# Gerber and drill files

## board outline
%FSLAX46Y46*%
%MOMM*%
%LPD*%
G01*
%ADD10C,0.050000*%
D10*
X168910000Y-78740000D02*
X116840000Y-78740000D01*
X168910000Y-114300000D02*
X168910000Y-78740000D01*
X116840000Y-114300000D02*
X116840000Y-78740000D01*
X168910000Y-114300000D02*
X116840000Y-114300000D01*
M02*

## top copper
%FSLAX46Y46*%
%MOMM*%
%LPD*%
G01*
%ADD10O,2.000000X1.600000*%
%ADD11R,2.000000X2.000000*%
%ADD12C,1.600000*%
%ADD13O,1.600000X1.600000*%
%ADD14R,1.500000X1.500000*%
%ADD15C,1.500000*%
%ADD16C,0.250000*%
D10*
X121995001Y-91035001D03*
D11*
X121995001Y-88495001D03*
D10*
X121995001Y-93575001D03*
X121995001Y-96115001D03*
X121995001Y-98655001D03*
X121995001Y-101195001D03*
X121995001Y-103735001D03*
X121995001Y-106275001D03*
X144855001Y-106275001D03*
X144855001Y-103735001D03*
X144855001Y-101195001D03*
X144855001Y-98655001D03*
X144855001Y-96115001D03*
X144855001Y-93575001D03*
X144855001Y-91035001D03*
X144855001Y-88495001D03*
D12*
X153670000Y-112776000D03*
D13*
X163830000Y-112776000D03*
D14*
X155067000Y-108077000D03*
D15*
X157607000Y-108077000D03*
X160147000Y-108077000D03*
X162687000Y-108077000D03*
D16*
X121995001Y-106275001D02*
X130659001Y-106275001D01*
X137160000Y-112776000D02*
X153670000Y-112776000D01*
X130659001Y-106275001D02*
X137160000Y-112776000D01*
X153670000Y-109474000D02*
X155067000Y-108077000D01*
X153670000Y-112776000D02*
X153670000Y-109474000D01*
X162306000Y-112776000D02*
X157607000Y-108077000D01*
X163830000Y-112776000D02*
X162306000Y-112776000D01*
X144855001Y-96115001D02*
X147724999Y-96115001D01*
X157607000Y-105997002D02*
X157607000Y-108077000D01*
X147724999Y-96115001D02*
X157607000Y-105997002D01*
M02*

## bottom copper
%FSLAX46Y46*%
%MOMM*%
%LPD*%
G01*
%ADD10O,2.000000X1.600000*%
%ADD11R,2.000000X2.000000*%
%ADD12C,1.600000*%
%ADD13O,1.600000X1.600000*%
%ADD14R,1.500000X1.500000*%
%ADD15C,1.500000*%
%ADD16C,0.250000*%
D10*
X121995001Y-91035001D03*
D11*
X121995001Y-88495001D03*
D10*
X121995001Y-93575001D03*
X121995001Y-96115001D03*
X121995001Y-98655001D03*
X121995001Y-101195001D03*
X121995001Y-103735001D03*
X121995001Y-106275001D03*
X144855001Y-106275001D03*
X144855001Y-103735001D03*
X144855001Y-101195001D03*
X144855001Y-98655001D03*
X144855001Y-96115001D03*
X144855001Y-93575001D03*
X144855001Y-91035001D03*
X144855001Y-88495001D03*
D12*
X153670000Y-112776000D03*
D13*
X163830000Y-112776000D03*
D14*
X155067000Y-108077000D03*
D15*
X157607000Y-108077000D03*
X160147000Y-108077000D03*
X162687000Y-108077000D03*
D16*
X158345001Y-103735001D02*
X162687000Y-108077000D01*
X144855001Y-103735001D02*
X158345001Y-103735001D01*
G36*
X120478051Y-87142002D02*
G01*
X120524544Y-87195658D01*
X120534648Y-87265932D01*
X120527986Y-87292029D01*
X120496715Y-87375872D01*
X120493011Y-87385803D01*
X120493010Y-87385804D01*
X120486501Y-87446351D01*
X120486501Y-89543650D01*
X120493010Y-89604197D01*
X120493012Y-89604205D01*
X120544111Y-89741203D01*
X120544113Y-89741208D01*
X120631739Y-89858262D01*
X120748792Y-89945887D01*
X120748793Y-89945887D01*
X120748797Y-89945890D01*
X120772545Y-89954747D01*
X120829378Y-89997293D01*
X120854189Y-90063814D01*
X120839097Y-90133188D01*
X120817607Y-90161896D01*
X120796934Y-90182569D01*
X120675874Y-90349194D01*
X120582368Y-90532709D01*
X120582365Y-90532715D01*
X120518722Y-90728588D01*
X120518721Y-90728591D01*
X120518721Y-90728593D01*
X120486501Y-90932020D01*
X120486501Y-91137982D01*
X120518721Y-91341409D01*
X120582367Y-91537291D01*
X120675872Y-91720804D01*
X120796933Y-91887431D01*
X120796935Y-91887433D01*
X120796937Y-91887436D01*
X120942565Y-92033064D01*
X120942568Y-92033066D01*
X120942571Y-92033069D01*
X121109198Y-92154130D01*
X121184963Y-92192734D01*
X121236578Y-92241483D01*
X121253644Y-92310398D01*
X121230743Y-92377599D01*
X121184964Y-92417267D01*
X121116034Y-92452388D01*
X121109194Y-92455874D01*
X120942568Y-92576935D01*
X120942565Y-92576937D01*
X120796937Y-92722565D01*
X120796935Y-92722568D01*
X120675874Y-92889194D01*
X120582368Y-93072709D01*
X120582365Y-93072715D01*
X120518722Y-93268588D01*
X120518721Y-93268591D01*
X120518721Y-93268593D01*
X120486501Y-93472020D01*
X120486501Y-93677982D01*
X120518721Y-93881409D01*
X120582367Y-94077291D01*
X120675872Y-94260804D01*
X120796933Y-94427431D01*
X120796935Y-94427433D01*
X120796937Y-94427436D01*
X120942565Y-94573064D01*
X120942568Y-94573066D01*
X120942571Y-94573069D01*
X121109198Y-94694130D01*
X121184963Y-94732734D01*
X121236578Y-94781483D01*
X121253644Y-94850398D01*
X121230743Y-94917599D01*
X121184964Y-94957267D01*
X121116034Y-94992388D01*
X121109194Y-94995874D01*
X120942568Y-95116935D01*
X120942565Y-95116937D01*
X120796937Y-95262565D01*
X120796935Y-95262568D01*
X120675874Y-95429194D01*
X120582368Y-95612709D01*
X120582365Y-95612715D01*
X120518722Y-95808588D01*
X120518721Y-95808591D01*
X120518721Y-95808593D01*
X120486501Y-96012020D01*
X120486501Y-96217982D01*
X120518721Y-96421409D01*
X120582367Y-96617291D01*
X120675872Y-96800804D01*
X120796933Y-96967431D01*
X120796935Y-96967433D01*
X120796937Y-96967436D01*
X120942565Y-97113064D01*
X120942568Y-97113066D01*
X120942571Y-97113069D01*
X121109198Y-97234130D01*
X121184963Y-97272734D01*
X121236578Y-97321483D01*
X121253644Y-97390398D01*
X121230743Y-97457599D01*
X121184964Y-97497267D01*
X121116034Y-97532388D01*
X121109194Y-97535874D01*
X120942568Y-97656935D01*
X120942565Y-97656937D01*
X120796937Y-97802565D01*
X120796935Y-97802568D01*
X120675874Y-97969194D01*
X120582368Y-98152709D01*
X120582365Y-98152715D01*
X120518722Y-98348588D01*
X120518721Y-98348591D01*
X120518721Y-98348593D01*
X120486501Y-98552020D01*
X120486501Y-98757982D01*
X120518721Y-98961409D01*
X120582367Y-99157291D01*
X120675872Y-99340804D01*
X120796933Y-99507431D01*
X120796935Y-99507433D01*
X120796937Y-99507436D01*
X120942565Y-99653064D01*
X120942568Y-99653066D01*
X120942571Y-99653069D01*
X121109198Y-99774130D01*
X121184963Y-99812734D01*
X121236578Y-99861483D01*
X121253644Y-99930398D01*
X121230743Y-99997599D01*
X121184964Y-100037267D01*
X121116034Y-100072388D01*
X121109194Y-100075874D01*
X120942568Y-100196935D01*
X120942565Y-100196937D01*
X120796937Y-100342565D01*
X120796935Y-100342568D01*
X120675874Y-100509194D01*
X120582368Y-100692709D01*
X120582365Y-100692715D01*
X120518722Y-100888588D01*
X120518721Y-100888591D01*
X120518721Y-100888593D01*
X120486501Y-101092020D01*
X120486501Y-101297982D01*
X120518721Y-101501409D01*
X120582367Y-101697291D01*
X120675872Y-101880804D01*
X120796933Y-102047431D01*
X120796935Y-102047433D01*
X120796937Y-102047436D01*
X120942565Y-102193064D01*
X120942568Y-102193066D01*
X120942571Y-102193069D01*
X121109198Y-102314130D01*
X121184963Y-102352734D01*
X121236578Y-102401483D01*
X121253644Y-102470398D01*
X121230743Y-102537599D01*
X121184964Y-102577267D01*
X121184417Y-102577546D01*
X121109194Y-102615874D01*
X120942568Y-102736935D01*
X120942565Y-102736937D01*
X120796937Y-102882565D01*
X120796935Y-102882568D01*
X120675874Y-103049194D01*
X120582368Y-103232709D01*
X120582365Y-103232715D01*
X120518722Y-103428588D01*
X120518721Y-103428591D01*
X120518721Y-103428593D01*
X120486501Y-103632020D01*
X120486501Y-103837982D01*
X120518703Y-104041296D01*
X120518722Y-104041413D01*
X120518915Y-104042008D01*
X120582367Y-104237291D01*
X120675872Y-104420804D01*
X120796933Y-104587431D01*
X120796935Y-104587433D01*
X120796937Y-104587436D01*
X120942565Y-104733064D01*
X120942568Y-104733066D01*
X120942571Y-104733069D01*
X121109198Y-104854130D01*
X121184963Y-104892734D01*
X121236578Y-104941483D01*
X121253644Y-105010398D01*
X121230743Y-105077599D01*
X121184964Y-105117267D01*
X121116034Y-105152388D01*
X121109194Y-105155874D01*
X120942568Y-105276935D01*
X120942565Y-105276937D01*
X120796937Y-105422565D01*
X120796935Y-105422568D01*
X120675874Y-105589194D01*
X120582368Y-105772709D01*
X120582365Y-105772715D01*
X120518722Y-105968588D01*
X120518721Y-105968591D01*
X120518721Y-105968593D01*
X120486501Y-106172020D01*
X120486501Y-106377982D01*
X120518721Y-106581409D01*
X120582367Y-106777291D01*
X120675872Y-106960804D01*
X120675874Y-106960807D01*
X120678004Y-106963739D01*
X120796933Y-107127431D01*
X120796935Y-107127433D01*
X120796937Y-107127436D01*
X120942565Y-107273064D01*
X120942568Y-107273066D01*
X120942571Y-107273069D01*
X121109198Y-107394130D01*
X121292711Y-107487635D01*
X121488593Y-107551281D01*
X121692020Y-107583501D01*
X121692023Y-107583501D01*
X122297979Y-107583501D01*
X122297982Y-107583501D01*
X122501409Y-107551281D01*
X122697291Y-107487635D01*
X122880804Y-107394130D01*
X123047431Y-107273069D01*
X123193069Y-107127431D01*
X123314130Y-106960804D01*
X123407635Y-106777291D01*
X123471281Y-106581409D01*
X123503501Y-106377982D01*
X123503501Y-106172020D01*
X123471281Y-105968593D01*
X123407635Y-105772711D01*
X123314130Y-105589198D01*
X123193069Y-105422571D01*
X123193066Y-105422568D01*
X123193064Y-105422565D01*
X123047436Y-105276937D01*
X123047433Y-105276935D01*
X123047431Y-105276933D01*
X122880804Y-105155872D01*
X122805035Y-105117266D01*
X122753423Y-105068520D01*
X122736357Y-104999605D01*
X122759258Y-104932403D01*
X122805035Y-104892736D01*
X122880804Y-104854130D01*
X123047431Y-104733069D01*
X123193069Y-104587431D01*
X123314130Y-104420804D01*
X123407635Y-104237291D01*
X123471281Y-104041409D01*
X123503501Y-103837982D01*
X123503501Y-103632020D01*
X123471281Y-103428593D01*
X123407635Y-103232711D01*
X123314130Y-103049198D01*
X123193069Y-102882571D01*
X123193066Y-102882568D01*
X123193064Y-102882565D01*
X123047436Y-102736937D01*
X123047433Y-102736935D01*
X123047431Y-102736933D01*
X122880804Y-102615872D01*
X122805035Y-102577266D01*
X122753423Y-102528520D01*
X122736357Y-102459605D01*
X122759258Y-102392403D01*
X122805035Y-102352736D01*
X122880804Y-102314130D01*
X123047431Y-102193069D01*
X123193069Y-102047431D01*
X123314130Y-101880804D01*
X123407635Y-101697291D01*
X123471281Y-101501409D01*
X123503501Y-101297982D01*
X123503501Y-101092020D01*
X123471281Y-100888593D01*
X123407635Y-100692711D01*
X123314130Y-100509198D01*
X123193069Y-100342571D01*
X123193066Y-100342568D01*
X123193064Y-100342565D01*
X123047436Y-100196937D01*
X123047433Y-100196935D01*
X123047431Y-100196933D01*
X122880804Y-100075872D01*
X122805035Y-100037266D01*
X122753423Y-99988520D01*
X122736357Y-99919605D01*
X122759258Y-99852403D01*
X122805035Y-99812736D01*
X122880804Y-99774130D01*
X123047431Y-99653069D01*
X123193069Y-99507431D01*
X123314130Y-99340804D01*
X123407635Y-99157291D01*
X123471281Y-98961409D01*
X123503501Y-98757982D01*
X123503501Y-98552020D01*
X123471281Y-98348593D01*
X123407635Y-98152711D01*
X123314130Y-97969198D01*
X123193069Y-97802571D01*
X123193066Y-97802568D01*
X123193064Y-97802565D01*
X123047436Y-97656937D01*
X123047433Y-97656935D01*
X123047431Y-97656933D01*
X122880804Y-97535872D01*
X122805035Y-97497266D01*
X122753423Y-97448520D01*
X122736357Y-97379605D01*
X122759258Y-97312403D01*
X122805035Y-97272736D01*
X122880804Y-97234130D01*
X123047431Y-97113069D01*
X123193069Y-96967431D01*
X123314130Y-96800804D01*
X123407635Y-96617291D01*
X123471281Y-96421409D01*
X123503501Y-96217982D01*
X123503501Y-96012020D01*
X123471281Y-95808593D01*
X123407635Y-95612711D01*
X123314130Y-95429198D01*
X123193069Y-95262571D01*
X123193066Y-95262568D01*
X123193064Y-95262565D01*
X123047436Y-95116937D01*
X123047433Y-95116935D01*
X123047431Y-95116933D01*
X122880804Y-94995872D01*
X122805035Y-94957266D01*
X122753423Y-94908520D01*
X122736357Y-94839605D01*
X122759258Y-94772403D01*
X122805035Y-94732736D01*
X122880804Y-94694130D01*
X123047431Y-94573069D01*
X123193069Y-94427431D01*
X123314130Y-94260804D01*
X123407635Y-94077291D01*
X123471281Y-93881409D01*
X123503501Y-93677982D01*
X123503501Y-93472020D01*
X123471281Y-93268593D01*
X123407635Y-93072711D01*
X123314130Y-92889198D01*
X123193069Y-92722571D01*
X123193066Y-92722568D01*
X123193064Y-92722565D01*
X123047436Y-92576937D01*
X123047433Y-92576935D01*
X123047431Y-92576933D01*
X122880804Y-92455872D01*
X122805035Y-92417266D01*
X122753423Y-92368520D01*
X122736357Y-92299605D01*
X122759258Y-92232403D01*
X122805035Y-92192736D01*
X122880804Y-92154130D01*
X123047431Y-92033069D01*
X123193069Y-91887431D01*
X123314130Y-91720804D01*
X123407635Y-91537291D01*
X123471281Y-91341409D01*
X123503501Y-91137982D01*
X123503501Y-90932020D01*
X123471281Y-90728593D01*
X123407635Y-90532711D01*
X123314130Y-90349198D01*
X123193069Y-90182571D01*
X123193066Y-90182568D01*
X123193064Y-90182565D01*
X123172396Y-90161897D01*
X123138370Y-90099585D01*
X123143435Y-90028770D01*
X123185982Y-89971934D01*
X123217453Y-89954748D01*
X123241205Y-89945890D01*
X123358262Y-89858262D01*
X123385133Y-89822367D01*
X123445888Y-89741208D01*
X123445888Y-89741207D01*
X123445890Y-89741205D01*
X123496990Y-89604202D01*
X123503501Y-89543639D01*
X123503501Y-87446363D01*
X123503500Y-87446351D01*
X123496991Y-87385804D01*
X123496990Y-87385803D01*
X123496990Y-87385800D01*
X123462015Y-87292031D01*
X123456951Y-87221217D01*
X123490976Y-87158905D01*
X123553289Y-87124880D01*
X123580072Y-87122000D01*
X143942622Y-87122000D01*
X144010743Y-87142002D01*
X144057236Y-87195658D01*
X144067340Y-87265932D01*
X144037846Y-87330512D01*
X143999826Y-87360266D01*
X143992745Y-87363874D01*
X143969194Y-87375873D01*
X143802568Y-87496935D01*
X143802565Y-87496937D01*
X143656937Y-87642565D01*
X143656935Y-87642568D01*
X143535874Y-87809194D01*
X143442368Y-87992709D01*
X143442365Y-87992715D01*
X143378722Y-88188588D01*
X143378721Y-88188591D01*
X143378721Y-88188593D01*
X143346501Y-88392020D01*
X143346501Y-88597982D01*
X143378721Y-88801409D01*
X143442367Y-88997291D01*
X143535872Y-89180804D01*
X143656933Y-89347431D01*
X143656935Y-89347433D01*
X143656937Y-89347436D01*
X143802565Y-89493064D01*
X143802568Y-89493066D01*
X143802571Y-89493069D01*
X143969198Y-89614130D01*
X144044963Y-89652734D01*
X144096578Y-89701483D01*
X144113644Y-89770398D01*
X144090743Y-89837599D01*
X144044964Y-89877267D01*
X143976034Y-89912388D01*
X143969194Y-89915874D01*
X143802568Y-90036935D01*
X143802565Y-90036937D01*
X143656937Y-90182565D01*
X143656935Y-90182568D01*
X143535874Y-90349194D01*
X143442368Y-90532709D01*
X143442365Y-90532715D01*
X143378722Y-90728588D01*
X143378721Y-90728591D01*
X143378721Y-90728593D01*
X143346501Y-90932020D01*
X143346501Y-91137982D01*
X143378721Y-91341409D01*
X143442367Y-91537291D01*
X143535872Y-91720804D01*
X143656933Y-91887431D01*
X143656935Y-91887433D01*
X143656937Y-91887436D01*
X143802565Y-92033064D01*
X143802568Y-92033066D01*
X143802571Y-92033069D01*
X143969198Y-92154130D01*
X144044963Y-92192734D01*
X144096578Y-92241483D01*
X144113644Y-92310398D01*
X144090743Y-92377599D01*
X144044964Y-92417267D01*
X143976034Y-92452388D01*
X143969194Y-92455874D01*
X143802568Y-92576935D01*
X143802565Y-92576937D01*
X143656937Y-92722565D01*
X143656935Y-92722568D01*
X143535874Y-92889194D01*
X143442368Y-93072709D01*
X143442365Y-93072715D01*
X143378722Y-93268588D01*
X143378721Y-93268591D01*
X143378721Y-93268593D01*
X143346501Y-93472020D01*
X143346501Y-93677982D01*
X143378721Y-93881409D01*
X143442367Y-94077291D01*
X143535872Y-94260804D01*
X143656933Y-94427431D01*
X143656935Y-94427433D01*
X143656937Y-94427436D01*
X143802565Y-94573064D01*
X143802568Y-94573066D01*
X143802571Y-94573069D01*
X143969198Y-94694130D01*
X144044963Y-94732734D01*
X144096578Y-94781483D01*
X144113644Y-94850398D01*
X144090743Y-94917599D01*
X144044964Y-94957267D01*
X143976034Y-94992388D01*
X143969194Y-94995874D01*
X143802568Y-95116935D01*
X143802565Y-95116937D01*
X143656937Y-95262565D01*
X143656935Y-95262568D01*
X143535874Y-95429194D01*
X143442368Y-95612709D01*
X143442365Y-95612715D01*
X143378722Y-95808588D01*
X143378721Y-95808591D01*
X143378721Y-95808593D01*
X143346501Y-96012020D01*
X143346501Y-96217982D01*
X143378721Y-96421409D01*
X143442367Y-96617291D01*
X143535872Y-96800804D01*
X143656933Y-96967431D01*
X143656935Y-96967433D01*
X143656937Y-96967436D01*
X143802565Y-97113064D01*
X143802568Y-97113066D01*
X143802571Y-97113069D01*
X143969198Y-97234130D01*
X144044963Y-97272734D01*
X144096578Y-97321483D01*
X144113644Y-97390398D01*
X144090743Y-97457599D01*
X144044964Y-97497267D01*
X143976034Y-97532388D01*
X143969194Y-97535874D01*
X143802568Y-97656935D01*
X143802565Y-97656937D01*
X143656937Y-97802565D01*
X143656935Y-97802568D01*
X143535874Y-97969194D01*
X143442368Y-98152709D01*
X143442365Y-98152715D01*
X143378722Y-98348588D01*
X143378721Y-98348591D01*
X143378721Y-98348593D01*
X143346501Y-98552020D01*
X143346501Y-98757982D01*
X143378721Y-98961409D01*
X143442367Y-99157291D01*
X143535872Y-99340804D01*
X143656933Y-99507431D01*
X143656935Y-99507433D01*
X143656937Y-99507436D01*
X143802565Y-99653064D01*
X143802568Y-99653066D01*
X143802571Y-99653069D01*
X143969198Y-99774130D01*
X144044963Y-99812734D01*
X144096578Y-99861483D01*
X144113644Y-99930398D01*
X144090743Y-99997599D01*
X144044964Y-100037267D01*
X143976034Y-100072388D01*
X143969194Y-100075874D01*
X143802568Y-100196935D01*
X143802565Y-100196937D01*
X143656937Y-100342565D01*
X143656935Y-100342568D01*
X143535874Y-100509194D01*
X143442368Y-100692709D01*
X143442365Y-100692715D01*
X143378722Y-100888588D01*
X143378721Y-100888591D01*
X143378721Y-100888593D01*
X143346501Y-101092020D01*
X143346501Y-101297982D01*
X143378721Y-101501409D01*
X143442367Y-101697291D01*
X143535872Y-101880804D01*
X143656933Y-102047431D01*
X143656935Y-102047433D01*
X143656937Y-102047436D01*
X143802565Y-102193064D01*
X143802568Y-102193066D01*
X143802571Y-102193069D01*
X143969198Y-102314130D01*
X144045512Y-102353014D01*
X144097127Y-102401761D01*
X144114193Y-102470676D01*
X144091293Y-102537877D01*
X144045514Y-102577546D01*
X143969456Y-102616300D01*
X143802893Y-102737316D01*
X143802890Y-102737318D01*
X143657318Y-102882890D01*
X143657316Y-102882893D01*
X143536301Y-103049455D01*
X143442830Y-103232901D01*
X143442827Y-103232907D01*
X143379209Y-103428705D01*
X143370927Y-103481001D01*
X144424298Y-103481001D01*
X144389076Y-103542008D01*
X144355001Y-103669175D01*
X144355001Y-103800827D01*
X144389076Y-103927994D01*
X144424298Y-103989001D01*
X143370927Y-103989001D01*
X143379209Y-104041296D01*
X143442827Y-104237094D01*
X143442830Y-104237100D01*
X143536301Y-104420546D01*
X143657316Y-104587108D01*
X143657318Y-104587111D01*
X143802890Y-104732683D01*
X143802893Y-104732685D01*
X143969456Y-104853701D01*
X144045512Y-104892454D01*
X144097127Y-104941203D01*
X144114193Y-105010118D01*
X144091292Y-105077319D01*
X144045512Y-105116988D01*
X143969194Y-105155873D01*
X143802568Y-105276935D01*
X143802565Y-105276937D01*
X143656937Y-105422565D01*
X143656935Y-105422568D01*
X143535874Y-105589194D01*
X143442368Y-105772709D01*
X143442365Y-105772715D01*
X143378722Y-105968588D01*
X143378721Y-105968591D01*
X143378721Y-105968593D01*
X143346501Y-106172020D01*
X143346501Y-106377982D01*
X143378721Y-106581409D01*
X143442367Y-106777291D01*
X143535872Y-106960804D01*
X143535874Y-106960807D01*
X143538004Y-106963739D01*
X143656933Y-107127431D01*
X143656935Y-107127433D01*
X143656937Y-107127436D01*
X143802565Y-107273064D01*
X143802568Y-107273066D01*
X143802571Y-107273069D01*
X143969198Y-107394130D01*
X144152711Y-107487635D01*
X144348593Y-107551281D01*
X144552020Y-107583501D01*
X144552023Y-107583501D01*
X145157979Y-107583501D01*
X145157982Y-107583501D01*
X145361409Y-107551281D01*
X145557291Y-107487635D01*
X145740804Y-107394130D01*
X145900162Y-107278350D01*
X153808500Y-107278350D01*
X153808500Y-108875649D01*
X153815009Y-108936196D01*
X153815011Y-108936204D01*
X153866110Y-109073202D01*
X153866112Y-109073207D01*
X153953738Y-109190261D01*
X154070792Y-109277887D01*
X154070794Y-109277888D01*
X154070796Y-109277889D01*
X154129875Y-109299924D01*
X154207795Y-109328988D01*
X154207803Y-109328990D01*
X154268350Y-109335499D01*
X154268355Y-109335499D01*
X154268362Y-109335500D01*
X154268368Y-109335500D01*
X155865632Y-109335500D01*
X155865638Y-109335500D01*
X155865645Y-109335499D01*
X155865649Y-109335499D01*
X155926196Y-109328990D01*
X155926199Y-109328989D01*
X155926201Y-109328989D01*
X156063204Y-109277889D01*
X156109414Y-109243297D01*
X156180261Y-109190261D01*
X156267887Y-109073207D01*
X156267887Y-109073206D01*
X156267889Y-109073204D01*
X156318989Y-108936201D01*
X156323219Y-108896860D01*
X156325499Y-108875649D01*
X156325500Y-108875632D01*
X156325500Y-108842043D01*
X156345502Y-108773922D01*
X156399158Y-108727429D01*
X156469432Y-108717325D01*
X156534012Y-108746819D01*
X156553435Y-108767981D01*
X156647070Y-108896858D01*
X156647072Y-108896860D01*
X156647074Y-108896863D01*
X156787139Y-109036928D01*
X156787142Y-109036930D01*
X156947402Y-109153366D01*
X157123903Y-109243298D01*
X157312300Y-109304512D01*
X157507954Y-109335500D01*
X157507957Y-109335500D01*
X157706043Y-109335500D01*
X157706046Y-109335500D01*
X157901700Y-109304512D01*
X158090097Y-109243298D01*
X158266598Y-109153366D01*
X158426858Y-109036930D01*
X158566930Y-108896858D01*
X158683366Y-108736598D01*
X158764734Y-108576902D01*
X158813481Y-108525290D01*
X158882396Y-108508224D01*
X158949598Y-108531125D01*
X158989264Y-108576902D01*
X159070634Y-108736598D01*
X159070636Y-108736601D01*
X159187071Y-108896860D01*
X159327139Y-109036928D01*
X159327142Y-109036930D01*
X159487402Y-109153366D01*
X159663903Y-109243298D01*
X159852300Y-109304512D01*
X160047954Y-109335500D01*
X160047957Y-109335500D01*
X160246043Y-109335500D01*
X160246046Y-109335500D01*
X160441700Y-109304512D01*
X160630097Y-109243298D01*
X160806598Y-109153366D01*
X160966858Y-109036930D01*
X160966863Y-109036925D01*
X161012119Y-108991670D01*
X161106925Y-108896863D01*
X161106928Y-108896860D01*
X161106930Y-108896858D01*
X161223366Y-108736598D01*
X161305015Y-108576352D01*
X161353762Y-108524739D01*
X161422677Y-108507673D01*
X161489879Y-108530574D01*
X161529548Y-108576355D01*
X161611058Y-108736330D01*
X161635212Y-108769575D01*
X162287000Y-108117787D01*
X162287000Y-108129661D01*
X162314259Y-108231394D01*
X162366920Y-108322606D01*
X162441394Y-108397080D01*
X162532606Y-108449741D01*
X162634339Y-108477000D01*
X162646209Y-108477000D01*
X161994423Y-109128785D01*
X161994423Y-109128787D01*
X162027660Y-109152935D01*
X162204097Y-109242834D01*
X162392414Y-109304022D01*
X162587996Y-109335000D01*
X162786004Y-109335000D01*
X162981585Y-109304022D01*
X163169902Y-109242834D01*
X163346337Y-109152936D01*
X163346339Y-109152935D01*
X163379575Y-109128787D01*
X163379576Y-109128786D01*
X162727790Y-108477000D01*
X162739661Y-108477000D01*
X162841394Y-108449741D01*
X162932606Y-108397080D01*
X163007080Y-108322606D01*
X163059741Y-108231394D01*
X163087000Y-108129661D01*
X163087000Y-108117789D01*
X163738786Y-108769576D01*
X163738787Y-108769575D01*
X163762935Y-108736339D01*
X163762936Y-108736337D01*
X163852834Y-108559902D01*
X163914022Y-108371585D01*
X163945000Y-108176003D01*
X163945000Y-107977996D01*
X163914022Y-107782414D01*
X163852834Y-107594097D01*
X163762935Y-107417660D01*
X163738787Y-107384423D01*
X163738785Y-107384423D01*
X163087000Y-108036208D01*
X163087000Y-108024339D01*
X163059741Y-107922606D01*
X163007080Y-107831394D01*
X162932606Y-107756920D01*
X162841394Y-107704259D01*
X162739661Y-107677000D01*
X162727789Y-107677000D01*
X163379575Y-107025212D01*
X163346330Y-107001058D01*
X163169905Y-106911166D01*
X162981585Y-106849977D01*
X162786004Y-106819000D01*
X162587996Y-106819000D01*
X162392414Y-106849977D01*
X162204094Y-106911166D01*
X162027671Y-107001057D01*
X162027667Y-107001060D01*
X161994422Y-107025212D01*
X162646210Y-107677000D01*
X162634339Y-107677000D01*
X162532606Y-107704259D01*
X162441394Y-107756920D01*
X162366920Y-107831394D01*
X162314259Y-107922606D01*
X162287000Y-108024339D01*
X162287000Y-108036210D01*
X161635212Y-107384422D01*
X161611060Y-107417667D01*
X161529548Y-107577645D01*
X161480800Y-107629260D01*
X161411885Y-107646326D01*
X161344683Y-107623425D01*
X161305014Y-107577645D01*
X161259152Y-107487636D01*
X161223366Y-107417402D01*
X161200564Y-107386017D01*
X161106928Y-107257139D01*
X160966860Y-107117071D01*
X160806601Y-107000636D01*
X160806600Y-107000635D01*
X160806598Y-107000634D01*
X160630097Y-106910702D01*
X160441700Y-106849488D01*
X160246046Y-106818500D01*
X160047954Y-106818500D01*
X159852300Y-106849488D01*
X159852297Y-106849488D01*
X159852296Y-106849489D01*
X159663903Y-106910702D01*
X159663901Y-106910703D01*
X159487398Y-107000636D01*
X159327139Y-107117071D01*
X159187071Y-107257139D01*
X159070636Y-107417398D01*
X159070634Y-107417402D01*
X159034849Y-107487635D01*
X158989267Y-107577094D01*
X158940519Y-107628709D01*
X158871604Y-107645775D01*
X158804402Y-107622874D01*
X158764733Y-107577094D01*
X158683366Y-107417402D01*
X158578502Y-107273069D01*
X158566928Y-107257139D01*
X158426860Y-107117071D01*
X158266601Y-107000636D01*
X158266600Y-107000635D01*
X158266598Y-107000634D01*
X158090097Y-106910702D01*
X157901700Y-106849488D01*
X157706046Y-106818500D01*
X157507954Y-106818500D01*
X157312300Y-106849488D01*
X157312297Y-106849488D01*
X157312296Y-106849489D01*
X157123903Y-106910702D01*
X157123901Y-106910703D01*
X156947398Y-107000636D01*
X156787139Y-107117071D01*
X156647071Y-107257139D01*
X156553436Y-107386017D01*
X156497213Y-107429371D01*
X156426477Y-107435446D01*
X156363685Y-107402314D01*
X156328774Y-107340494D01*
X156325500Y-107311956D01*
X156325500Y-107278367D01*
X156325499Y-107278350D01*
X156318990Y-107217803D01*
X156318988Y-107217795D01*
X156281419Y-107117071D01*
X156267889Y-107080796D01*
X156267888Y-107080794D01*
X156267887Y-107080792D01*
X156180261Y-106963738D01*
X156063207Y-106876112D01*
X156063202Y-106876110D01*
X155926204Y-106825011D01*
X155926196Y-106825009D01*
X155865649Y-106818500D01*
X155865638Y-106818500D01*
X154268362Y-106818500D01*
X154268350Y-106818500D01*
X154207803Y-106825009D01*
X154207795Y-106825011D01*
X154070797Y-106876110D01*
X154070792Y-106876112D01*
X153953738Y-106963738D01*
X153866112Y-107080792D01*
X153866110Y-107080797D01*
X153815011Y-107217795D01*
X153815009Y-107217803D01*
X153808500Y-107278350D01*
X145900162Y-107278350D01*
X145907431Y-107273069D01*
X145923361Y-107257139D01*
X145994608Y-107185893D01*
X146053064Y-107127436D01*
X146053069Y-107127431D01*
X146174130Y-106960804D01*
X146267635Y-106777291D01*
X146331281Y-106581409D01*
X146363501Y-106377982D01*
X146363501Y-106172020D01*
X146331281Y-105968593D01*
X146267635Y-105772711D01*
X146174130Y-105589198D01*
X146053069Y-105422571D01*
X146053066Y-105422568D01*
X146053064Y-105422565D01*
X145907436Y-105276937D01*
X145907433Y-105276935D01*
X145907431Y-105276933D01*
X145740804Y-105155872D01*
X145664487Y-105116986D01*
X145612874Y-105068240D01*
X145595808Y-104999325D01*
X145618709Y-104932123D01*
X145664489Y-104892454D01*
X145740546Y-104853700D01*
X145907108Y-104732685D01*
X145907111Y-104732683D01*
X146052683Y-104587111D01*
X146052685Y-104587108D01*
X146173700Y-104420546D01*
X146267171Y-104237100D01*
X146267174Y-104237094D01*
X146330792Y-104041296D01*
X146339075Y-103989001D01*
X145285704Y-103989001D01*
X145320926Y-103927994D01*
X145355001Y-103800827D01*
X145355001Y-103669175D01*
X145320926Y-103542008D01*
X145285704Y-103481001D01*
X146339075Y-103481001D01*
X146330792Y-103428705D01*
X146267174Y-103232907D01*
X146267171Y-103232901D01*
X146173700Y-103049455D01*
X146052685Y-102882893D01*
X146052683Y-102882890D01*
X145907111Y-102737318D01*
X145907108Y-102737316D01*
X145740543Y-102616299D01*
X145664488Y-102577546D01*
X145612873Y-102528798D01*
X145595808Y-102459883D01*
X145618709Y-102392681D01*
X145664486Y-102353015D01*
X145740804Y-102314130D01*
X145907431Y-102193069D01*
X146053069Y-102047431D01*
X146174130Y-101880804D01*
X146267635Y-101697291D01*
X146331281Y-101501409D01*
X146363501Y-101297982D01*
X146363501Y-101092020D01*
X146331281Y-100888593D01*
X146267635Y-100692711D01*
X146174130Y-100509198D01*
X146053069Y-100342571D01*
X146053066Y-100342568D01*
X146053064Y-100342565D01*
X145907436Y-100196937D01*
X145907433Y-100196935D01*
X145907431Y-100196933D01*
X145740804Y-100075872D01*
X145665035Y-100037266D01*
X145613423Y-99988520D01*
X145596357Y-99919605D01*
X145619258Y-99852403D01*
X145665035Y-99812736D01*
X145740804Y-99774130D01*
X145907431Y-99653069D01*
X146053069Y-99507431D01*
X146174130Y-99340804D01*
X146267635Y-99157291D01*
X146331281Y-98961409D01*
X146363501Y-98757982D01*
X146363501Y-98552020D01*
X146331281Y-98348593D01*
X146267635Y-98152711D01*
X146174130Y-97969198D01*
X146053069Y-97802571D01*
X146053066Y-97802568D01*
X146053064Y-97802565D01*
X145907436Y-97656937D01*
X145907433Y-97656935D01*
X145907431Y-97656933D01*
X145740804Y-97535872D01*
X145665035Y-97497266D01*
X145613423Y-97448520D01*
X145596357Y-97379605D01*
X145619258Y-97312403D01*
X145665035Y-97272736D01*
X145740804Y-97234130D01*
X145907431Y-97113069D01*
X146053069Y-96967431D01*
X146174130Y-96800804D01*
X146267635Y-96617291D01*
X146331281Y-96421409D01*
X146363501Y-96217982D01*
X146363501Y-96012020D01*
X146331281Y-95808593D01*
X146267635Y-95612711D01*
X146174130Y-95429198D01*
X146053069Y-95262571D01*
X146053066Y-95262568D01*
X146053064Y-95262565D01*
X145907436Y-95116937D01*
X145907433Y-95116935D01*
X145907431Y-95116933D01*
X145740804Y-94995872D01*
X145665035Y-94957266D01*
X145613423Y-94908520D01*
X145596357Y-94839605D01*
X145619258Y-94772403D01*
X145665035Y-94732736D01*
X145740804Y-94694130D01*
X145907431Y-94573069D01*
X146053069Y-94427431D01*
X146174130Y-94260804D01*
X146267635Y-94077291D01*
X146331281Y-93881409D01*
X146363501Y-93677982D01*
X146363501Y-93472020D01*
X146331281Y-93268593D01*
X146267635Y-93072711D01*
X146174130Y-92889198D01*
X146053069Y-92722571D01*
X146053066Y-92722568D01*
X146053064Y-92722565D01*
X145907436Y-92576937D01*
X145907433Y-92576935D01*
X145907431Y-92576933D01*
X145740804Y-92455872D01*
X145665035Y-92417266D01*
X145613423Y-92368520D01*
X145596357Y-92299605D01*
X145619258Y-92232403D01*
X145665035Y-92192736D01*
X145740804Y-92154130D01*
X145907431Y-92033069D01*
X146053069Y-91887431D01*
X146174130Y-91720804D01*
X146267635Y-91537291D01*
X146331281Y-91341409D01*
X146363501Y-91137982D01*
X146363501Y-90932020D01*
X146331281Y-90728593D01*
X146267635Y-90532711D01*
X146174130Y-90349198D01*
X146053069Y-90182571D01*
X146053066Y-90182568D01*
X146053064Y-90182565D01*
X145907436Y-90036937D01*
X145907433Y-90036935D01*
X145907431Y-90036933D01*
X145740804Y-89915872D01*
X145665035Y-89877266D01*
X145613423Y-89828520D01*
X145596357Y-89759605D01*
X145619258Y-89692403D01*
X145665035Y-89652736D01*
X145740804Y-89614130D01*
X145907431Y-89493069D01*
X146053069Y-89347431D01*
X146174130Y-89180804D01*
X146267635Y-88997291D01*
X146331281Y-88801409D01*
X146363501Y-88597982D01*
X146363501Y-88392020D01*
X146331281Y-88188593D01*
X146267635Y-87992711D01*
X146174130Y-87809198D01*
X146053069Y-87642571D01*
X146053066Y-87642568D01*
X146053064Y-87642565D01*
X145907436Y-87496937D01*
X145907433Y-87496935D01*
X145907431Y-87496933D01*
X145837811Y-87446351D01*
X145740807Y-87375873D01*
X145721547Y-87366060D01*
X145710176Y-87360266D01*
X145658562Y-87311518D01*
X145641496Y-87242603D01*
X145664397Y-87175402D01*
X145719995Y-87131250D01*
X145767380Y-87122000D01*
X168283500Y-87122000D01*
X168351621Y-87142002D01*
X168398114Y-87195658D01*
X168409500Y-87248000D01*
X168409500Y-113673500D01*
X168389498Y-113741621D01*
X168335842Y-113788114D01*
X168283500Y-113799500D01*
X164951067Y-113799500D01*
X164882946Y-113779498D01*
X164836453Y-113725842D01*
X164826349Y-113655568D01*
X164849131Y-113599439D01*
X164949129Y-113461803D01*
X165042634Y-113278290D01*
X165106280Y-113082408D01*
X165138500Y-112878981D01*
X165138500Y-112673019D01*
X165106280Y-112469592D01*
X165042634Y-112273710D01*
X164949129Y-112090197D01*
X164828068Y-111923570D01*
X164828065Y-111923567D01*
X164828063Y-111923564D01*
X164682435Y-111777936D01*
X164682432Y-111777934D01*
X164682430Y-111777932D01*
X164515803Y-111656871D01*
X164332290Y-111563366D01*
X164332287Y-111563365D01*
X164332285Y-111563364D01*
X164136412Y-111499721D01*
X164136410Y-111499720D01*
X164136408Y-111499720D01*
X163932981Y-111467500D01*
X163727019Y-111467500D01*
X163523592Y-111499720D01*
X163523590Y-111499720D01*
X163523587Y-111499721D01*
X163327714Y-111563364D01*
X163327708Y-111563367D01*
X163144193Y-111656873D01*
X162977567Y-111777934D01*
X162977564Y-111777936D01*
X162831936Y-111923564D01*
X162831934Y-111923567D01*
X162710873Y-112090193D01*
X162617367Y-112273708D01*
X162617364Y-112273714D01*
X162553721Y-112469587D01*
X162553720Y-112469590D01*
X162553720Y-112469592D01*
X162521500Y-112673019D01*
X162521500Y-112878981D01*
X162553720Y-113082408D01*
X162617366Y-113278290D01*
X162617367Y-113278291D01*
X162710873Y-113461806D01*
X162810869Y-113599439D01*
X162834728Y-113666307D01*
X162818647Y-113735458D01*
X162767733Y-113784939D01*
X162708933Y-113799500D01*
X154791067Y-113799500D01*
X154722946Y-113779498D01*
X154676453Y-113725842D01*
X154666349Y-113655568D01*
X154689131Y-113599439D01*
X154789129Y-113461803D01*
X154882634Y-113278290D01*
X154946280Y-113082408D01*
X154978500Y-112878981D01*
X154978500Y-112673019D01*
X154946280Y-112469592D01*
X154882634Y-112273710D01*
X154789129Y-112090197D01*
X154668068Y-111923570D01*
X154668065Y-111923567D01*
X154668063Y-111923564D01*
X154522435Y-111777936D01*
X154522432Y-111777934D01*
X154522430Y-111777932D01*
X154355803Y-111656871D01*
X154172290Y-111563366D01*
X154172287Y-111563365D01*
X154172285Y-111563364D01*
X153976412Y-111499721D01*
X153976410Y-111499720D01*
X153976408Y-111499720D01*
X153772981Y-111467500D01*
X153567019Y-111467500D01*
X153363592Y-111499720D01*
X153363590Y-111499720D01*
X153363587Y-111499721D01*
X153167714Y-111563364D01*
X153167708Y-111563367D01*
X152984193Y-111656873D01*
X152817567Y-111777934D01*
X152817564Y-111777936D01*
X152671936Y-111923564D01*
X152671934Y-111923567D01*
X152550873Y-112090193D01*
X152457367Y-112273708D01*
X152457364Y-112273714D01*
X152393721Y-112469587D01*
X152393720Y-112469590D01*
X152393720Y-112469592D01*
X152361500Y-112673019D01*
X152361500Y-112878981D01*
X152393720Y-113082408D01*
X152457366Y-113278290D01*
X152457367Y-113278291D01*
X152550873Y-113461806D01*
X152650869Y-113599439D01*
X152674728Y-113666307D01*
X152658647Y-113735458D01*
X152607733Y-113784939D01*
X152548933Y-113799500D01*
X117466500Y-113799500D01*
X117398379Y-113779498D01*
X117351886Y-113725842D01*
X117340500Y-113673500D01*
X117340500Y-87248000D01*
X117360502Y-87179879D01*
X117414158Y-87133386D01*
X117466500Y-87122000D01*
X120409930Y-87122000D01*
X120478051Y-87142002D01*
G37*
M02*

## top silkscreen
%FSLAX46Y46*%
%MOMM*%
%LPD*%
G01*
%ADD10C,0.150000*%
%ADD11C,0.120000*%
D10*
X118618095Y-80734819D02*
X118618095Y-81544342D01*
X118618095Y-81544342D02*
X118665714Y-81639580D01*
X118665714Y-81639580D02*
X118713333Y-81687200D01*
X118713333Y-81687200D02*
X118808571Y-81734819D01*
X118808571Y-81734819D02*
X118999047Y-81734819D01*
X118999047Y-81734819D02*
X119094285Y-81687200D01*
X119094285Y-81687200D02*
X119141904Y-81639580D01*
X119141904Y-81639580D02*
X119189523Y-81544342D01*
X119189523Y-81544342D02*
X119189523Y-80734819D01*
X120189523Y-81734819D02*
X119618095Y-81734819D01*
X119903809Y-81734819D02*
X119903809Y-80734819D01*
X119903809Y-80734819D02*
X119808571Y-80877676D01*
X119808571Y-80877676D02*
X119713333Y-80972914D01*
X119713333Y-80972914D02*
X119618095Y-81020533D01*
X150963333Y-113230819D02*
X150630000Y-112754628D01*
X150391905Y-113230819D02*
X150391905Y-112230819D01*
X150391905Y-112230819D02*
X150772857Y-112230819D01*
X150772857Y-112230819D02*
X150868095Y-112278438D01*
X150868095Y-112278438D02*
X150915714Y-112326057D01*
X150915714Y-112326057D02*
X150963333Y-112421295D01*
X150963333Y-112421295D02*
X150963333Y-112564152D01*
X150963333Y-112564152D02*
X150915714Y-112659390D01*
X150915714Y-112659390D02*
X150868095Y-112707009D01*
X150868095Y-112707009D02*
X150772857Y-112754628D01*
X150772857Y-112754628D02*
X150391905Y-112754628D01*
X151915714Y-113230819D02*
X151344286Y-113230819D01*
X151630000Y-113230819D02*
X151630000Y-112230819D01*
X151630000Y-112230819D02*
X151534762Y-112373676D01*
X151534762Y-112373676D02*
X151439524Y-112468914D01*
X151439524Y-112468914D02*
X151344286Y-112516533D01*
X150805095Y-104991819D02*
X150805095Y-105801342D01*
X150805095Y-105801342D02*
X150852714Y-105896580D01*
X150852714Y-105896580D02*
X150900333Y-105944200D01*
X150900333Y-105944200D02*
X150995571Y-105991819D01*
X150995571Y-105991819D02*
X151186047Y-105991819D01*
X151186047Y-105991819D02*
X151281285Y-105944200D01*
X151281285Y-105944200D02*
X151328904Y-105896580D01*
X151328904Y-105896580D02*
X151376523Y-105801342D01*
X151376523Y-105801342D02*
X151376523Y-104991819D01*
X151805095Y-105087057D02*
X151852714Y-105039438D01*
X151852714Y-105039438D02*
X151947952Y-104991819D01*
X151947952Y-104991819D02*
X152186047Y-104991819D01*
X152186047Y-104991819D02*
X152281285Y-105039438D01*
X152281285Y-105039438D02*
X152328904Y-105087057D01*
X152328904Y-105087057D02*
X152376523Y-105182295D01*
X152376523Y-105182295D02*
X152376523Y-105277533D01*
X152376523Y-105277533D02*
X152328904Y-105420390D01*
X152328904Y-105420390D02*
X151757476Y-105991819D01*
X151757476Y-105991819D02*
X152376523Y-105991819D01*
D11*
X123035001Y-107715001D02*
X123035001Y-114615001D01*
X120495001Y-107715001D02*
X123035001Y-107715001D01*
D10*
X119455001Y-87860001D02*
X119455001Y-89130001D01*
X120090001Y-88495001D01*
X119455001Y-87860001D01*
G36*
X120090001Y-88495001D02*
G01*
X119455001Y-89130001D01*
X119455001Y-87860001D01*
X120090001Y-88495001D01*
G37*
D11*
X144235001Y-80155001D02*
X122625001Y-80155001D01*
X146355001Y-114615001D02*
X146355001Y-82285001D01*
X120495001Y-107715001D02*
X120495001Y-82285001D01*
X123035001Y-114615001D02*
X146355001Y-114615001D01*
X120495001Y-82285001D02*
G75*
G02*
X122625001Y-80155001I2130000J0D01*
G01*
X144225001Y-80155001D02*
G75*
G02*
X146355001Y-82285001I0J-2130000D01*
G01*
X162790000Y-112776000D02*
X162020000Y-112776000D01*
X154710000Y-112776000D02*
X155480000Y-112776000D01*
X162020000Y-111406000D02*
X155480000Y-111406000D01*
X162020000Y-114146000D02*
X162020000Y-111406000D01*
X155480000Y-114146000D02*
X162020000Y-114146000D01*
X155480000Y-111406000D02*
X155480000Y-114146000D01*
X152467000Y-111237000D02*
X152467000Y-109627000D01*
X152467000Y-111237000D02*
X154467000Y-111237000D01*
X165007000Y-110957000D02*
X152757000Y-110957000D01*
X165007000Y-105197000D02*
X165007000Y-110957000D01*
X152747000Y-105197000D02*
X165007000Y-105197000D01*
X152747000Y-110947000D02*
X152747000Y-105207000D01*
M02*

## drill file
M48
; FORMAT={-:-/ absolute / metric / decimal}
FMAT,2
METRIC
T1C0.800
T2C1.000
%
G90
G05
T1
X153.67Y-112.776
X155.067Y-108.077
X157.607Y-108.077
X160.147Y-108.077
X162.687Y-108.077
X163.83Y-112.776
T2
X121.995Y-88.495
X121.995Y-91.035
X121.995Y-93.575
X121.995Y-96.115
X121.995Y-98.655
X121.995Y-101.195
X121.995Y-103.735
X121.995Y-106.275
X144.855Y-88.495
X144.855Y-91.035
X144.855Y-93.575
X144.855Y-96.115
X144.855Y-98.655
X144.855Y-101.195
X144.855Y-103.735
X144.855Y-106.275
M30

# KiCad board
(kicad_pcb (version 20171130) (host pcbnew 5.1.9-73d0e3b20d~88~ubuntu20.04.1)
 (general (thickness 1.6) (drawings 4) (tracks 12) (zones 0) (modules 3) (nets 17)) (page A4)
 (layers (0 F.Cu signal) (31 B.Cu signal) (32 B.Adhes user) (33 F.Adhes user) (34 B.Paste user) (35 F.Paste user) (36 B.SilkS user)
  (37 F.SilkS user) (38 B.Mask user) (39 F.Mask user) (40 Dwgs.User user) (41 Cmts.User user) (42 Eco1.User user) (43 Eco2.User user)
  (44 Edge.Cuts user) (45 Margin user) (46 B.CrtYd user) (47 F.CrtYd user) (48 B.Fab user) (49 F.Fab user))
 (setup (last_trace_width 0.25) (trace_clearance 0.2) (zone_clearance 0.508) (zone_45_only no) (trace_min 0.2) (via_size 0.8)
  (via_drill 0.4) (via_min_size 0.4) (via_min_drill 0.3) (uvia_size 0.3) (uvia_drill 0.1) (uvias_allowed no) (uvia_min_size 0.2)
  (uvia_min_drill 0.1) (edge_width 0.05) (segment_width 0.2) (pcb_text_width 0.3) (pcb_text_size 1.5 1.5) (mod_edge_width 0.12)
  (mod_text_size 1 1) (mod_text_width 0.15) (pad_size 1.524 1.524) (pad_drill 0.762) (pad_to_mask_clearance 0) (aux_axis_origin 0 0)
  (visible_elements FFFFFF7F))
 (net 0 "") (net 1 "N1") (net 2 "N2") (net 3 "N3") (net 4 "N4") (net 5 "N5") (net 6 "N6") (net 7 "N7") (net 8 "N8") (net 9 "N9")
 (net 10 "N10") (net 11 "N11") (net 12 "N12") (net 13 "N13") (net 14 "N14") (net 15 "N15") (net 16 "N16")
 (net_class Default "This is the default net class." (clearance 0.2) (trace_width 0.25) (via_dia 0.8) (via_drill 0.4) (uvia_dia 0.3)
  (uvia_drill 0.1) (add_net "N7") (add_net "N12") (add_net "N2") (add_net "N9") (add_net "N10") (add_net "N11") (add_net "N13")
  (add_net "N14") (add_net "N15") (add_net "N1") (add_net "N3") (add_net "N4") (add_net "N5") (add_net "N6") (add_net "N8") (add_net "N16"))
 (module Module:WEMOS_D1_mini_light (layer F.Cu) (at 121.995001 88.495001)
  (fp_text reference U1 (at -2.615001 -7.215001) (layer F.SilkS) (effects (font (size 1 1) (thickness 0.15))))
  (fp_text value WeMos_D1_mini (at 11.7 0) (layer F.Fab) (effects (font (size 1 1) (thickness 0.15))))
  (fp_line (start 1.04 19.22) (end 1.04 26.12) (layer F.SilkS) (width 0.12))
  (fp_line (start -1.5 19.22) (end 1.04 19.22) (layer F.SilkS) (width 0.12))
  (fp_poly (pts (xy -2.54 -0.635) (xy -2.54 0.635) (xy -1.905 0)) (layer F.SilkS) (width 0.15))
  (fp_line (start 22.24 -8.34) (end 0.63 -8.34) (layer F.SilkS) (width 0.12))
  (fp_line (start 24.36 26.12) (end 24.36 -6.21) (layer F.SilkS) (width 0.12))
  (fp_line (start -1.5 19.22) (end -1.5 -6.21) (layer F.SilkS) (width 0.12))
  (fp_line (start 1.04 26.12) (end 24.36 26.12) (layer F.SilkS) (width 0.12))
  (fp_arc (start 0.63 -6.21) (end 0.63 -8.34) (angle -90) (layer F.SilkS) (width 0.12))
  (fp_arc (start 22.23 -6.21) (end 24.36 -6.21) (angle -90) (layer F.SilkS) (width 0.12))
  (pad 2 thru_hole oval (at 0 2.54) (size 2 1.6) (drill 1) (layers *.Cu *.Mask) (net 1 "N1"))
  (pad 1 thru_hole rect (at 0 0) (size 2 2) (drill 1) (layers *.Cu *.Mask) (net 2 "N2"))
  (pad 3 thru_hole oval (at 0 5.08) (size 2 1.6) (drill 1) (layers *.Cu *.Mask) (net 2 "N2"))
  (pad 4 thru_hole oval (at 0 7.62) (size 2 1.6) (drill 1) (layers *.Cu *.Mask) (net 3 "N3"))
  (pad 5 thru_hole oval (at 0 10.16) (size 2 1.6) (drill 1) (layers *.Cu *.Mask) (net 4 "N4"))
  (pad 6 thru_hole oval (at 0 12.7) (size 2 1.6) (drill 1) (layers *.Cu *.Mask) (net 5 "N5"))
  (pad 7 thru_hole oval (at 0 15.24) (size 2 1.6) (drill 1) (layers *.Cu *.Mask) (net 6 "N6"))
  (pad 8 thru_hole oval (at 0 17.78) (size 2 1.6) (drill 1) (layers *.Cu *.Mask) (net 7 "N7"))
  (pad 9 thru_hole oval (at 22.86 17.78) (size 2 1.6) (drill 1) (layers *.Cu *.Mask) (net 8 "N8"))
  (pad 10 thru_hole oval (at 22.86 15.24) (size 2 1.6) (drill 1) (layers *.Cu *.Mask) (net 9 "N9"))
  (pad 11 thru_hole oval (at 22.86 12.7) (size 2 1.6) (drill 1) (layers *.Cu *.Mask) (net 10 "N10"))
  (pad 12 thru_hole oval (at 22.86 10.16) (size 2 1.6) (drill 1) (layers *.Cu *.Mask) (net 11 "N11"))
  (pad 13 thru_hole oval (at 22.86 7.62) (size 2 1.6) (drill 1) (layers *.Cu *.Mask) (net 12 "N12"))
  (pad 14 thru_hole oval (at 22.86 5.08) (size 2 1.6) (drill 1) (layers *.Cu *.Mask) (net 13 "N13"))
  (pad 15 thru_hole oval (at 22.86 2.54) (size 2 1.6) (drill 1) (layers *.Cu *.Mask) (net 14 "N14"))
  (pad 16 thru_hole oval (at 22.86 0) (size 2 1.6) (drill 1) (layers *.Cu *.Mask) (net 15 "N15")))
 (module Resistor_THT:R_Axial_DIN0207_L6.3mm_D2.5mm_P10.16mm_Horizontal (layer F.Cu) (at 153.67 112.776)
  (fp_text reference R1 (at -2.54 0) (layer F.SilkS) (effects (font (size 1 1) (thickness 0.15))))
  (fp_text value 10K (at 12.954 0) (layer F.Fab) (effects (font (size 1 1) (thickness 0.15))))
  (fp_line (start 9.12 0) (end 8.35 0) (layer F.SilkS) (width 0.12))
  (fp_line (start 1.04 0) (end 1.81 0) (layer F.SilkS) (width 0.12))
  (fp_line (start 8.35 -1.37) (end 1.81 -1.37) (layer F.SilkS) (width 0.12))
  (fp_line (start 8.35 1.37) (end 8.35 -1.37) (layer F.SilkS) (width 0.12))
  (fp_line (start 1.81 1.37) (end 8.35 1.37) (layer F.SilkS) (width 0.12))
  (fp_line (start 1.81 -1.37) (end 1.81 1.37) (layer F.SilkS) (width 0.12))
  (pad 1 thru_hole circle (at 0 0) (size 1.6 1.6) (drill 0.8) (layers *.Cu *.Mask) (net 7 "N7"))
  (pad 2 thru_hole oval (at 10.16 0) (size 1.6 1.6) (drill 0.8) (layers *.Cu *.Mask) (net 12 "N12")))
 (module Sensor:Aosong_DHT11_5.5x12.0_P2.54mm (layer F.Cu) (at 155.067 108.077 90)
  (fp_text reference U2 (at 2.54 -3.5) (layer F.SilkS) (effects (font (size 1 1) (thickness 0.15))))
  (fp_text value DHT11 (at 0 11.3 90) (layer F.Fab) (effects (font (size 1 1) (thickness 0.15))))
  (fp_line (start -3.16 -2.6) (end -1.55 -2.6) (layer F.SilkS) (width 0.12))
  (fp_line (start -3.16 -2.6) (end -3.16 -0.6) (layer F.SilkS) (width 0.12))
  (fp_line (start -2.88 9.94) (end -2.88 -2.31) (layer F.SilkS) (width 0.12))
  (fp_line (start 2.88 9.94) (end -2.88 9.94) (layer F.SilkS) (width 0.12))
  (fp_line (start 2.88 -2.32) (end 2.88 9.94) (layer F.SilkS) (width 0.12))
  (fp_line (start -2.87 -2.32) (end 2.87 -2.32) (layer F.SilkS) (width 0.12))
  (pad 1 thru_hole rect (at 0 0 90) (size 1.5 1.5) (drill 0.8) (layers *.Cu *.Mask) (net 7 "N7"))
  (pad 2 thru_hole circle (at 0 2.54 90) (size 1.5 1.5) (drill 0.8) (layers *.Cu *.Mask) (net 12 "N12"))
  (pad 3 thru_hole circle (at 0 5.08 90) (size 1.5 1.5) (drill 0.8) (layers *.Cu *.Mask) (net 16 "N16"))
  (pad 4 thru_hole circle (at 0 7.62 90) (size 1.5 1.5) (drill 0.8) (layers *.Cu *.Mask) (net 9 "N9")))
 (gr_line (start 168.91 78.74) (end 116.84 78.74) (layer Edge.Cuts) (width 0.05))
 (gr_line (start 168.91 114.3) (end 168.91 78.74) (layer Edge.Cuts) (width 0.05))
 (gr_line (start 116.84 114.3) (end 116.84 78.74) (layer Edge.Cuts) (width 0.05))
 (gr_line (start 168.91 114.3) (end 116.84 114.3) (layer Edge.Cuts) (width 0.05))
 (segment (start 121.995001 106.275001) (end 130.659001 106.275001) (width 0.25) (layer F.Cu) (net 7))
 (segment (start 137.16 112.776) (end 153.67 112.776) (width 0.25) (layer F.Cu) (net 7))
 (segment (start 130.659001 106.275001) (end 137.16 112.776) (width 0.25) (layer F.Cu) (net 7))
 (segment (start 153.67 109.474) (end 155.067 108.077) (width 0.25) (layer F.Cu) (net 7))
 (segment (start 153.67 112.776) (end 153.67 109.474) (width 0.25) (layer F.Cu) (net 7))
 (segment (start 162.306 112.776) (end 157.607 108.077) (width 0.25) (layer F.Cu) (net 12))
 (segment (start 163.83 112.776) (end 162.306 112.776) (width 0.25) (layer F.Cu) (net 12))
 (segment (start 144.855001 96.115001) (end 147.724999 96.115001) (width 0.25) (layer F.Cu) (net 12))
 (segment (start 157.607 105.997002) (end 157.607 108.077) (width 0.25) (layer F.Cu) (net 12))
 (segment (start 147.724999 96.115001) (end 157.607 105.997002) (width 0.25) (layer F.Cu) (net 12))
 (segment (start 158.345001 103.735001) (end 162.687 108.077) (width 0.25) (layer B.Cu) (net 9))
 (segment (start 144.855001 103.735001) (end 158.345001 103.735001) (width 0.25) (layer B.Cu) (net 9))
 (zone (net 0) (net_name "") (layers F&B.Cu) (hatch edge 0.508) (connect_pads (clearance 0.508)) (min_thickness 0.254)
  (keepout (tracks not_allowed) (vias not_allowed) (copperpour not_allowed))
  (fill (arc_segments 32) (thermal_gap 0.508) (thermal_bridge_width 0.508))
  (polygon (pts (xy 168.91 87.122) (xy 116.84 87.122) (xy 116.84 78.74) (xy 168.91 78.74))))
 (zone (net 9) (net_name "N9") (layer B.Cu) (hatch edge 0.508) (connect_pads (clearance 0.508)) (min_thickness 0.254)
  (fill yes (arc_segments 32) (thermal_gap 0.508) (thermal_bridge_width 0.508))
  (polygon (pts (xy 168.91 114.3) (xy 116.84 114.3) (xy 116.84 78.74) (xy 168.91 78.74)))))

